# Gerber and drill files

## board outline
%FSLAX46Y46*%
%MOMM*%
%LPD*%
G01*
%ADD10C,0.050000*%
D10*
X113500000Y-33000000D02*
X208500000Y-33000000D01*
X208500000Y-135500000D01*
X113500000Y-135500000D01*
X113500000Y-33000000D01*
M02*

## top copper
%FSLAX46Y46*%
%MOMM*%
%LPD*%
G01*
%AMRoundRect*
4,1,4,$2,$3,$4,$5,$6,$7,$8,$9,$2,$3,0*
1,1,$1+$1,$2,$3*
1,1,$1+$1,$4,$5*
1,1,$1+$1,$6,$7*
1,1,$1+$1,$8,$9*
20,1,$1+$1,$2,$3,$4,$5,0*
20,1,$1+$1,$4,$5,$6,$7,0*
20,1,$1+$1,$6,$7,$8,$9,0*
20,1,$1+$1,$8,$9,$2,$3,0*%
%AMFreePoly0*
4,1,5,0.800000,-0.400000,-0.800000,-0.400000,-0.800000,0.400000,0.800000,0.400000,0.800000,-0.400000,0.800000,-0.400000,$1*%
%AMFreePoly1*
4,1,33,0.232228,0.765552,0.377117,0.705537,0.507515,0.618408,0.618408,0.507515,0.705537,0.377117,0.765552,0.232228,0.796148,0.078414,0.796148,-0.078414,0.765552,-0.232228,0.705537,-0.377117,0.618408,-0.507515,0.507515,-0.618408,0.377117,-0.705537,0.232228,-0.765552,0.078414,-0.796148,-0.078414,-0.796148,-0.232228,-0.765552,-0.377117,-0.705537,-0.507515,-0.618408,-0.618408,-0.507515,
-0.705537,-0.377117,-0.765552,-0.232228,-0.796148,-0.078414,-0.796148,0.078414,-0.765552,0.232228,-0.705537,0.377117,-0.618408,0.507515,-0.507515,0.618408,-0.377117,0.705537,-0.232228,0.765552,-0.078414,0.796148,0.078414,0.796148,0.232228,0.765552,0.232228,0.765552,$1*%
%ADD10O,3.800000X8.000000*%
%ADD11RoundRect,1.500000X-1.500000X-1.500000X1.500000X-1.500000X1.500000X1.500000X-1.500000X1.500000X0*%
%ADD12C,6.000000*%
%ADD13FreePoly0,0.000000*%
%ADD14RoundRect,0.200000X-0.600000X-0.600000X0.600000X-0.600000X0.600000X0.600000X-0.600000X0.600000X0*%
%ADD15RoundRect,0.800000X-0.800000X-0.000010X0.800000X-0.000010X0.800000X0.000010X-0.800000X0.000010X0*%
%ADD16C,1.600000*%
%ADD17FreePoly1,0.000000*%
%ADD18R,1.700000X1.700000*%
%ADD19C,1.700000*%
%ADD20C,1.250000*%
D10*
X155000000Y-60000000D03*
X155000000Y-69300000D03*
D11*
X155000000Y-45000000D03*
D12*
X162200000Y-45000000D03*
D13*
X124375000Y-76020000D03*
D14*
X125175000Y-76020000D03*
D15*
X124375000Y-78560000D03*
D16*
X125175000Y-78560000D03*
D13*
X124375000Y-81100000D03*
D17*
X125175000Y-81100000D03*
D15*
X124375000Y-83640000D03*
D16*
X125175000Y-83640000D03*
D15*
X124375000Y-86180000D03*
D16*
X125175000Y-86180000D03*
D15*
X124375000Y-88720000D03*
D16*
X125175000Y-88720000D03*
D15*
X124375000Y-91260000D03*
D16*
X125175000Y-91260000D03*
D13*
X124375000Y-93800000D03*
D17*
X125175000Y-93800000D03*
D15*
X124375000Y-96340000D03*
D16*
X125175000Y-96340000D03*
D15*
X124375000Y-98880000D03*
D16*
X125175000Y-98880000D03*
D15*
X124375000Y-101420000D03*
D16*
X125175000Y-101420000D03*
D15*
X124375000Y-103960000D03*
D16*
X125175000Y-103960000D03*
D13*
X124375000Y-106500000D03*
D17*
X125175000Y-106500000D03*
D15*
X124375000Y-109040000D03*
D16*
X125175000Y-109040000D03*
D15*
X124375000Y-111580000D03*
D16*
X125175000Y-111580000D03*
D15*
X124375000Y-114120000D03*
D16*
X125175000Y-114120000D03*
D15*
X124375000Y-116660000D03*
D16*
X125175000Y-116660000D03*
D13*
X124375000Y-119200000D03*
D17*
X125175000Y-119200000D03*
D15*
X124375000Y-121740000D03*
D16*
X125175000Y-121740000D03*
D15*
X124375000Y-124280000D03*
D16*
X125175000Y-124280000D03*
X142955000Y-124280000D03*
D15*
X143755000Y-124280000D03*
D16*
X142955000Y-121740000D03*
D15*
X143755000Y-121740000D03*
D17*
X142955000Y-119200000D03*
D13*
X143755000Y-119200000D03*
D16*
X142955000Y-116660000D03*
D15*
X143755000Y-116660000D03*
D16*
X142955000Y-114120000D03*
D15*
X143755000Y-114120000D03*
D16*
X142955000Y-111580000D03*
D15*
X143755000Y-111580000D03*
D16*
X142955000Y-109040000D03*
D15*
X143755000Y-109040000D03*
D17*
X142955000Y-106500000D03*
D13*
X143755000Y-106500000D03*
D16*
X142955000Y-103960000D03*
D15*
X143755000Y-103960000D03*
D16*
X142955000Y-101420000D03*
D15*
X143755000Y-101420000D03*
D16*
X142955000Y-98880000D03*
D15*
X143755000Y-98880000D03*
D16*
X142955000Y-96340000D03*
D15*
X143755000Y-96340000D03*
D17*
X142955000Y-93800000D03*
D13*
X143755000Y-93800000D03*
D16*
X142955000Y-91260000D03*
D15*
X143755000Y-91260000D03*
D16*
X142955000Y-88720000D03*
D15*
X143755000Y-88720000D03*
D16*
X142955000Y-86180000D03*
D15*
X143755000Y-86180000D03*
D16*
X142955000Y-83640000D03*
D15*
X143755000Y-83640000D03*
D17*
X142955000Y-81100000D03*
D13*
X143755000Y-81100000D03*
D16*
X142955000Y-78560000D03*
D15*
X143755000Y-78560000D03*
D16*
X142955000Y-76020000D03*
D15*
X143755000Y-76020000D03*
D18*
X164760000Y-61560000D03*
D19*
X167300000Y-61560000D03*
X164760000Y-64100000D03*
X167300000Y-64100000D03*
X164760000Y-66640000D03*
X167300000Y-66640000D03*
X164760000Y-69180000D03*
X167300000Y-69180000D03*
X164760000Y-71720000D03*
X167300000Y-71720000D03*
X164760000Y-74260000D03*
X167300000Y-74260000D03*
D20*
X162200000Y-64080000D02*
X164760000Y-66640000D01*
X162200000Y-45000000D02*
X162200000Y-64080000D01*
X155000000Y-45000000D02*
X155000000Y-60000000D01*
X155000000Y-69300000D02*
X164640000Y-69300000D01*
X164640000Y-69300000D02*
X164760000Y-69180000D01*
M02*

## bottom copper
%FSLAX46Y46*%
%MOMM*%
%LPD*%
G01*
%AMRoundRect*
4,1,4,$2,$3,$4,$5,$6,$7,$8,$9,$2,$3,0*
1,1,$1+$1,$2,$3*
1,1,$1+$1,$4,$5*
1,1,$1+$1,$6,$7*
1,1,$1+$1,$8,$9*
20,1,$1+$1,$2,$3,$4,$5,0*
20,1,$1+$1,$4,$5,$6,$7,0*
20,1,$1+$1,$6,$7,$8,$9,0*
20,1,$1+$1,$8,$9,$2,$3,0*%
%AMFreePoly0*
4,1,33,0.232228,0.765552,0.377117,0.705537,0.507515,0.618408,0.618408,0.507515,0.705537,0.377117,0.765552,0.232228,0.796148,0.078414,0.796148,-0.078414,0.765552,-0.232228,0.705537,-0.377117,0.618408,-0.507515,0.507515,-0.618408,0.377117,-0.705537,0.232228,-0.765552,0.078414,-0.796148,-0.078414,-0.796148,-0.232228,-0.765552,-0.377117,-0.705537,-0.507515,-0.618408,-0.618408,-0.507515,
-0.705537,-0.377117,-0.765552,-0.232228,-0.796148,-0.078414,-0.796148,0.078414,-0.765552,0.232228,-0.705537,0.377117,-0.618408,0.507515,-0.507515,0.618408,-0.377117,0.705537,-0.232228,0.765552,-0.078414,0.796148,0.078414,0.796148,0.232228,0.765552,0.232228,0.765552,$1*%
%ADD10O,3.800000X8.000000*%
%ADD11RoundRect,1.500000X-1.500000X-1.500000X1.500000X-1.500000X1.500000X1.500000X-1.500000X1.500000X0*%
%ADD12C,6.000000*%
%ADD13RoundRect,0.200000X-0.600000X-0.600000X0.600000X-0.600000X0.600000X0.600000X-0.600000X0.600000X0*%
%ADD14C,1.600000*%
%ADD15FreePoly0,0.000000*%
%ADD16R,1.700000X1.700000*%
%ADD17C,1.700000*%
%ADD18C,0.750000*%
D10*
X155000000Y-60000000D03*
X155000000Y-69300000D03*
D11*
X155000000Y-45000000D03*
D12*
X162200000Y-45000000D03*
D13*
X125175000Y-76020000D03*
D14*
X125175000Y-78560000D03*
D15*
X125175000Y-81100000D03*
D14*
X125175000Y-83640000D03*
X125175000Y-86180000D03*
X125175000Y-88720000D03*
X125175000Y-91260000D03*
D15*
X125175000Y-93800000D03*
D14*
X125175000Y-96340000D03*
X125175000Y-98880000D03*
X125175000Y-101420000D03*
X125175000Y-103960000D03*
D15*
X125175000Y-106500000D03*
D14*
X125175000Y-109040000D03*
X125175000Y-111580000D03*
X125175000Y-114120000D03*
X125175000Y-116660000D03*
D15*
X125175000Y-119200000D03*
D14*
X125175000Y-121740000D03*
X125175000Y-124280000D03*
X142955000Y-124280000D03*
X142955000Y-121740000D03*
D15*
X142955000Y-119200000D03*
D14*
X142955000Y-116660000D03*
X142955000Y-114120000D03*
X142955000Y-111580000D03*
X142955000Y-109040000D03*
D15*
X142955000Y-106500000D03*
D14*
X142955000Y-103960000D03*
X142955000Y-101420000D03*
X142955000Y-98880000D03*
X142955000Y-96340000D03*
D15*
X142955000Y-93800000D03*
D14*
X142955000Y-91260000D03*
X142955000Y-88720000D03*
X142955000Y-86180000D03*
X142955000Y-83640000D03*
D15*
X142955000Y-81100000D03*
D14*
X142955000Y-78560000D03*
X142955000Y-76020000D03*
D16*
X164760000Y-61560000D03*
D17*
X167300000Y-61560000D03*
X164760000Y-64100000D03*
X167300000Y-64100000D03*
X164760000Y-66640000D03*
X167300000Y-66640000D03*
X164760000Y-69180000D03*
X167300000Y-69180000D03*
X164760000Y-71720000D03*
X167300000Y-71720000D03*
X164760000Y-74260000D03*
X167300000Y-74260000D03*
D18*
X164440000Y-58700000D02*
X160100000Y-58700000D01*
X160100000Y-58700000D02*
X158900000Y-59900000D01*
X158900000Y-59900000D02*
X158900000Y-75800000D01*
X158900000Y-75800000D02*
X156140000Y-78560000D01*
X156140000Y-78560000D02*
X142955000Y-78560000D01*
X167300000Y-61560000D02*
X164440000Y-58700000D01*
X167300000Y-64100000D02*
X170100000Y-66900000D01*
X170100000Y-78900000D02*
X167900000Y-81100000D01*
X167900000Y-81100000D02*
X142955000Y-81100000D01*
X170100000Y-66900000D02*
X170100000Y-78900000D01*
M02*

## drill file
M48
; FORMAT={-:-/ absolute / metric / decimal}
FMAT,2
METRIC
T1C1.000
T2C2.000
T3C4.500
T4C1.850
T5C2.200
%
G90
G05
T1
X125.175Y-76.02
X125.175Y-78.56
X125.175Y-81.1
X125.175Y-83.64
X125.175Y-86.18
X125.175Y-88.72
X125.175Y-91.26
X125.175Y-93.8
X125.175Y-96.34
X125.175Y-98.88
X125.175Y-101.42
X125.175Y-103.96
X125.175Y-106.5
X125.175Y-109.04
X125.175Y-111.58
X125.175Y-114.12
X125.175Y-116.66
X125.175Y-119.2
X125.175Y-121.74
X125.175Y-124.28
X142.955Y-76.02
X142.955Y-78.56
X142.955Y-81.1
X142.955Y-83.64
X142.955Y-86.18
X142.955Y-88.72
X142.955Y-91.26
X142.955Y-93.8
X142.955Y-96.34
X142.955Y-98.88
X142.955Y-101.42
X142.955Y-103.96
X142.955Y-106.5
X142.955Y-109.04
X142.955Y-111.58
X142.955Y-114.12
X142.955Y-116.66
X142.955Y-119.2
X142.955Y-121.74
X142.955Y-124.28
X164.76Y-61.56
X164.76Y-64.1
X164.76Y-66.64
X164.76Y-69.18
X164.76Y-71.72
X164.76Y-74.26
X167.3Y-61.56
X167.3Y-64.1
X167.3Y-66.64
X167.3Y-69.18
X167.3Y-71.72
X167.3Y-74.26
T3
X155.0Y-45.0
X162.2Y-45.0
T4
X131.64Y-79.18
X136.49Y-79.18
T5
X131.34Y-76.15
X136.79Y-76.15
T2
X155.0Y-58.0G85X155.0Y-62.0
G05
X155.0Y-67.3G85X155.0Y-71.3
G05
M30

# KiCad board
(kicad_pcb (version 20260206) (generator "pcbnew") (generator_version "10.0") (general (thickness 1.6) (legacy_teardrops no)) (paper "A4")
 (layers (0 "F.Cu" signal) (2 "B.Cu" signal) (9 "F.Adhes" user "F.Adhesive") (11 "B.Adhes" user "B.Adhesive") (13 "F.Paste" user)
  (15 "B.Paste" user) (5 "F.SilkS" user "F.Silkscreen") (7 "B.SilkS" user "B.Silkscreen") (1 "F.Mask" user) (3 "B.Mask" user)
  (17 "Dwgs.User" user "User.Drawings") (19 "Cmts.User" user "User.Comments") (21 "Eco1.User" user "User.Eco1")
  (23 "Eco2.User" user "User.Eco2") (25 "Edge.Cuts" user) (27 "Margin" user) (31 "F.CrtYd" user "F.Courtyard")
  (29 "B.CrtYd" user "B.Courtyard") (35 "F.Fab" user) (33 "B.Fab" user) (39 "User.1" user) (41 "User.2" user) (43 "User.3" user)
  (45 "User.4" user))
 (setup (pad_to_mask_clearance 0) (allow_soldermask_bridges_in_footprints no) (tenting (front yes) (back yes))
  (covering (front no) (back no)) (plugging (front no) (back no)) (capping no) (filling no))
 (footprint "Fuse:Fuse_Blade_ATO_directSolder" (layer "F.Cu") (at 155 60 -90)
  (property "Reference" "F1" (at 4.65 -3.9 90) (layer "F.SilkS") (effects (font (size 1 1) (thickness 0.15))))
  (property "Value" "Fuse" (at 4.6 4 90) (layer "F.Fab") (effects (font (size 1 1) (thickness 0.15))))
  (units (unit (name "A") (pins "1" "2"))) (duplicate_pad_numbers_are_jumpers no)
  (pad "1" thru_hole oval (at 0 0 270) (size 8 3.8) (drill oval 6 2) (layers "*.Cu" "*.Mask") (remove_unused_layers no) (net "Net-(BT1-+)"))
  (pad "2" thru_hole oval (at 9.3 0 270) (size 8 3.8) (drill oval 6 2) (layers "*.Cu" "*.Mask") (remove_unused_layers no)
   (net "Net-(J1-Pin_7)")))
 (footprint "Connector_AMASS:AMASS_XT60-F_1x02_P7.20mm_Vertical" (layer "F.Cu") (at 155 45)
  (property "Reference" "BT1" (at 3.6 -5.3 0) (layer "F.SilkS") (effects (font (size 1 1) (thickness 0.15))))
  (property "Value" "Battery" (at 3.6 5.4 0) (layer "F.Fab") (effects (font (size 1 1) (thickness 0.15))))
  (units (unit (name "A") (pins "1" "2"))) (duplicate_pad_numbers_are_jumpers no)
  (pad "1" thru_hole roundrect (at 0 0) (size 6 6) (drill 4.5) (layers "*.Cu" "*.Mask") (remove_unused_layers no) (roundrect_rratio 0.25)
   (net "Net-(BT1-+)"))
  (pad "2" thru_hole circle (at 7.2 0) (size 6 6) (drill 4.5) (layers "*.Cu" "*.Mask") (remove_unused_layers no) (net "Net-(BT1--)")))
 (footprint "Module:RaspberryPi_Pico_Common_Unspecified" (layer "F.Cu") (at 134.065 100.15)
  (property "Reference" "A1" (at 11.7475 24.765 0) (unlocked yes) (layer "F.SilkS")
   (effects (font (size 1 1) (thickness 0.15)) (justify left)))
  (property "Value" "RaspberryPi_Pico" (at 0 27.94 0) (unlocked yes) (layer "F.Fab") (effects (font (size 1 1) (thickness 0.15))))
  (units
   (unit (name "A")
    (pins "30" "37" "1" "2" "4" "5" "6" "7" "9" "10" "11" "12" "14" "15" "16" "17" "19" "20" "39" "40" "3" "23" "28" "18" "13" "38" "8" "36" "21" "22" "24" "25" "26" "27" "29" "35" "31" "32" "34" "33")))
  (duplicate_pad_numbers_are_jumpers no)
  (pad "" np_thru_hole circle (at -2.725 -24) (size 2.2 2.2) (drill 2.2) (layers "*.Mask"))
  (pad "" np_thru_hole circle (at -2.425 -20.97) (size 1.85 1.85) (drill 1.85) (layers "*.Mask"))
  (pad "" np_thru_hole circle (at 2.425 -20.97) (size 1.85 1.85) (drill 1.85) (layers "*.Mask"))
  (pad "" np_thru_hole circle (at 2.725 -24) (size 2.2 2.2) (drill 2.2) (layers "*.Mask"))
  (pad "1" smd custom (at -9.69 -24.13) (size 1.6 0.8) (layers "F.Cu" "F.Mask") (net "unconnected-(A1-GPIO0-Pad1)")
   (options (clearance outline) (anchor rect)) (primitives))
  (pad "1" thru_hole roundrect (at -8.89 -24.13) (size 1.6 1.6) (drill 1) (layers "*.Cu" "*.Mask") (remove_unused_layers no)
   (roundrect_rratio 0.125) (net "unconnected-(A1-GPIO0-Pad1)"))
  (pad "2" smd roundrect (at -9.69 -21.59) (size 3.2 1.6) (layers "F.Cu" "F.Mask") (roundrect_rratio 0.5)
   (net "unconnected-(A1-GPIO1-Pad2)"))
  (pad "2" thru_hole circle (at -8.89 -21.59) (size 1.6 1.6) (drill 1) (layers "*.Cu" "*.Mask") (remove_unused_layers no)
   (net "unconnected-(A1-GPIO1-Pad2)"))
  (pad "3" smd custom (at -9.69 -19.05) (size 1.6 0.8) (layers "F.Cu" "F.Mask") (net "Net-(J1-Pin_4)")
   (options (clearance outline) (anchor rect)) (primitives))
  (pad "3" thru_hole custom (at -8.89 -19.05) (size 1.6 1.6) (drill 1) (layers "*.Cu" "*.Mask") (remove_unused_layers no)
   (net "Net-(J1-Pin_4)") (options (clearance outline) (anchor circle)) (primitives))
  (pad "4" smd roundrect (at -9.69 -16.51) (size 3.2 1.6) (layers "F.Cu" "F.Mask") (roundrect_rratio 0.5)
   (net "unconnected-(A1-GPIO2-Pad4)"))
  (pad "4" thru_hole circle (at -8.89 -16.51) (size 1.6 1.6) (drill 1) (layers "*.Cu" "*.Mask") (remove_unused_layers no)
   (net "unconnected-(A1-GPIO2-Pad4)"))
  (pad "5" smd roundrect (at -9.69 -13.97) (size 3.2 1.6) (layers "F.Cu" "F.Mask") (roundrect_rratio 0.5)
   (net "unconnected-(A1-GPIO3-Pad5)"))
  (pad "5" thru_hole circle (at -8.89 -13.97) (size 1.6 1.6) (drill 1) (layers "*.Cu" "*.Mask") (remove_unused_layers no)
   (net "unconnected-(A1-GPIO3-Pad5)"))
  (pad "6" smd roundrect (at -9.69 -11.43) (size 3.2 1.6) (layers "F.Cu" "F.Mask") (roundrect_rratio 0.5)
   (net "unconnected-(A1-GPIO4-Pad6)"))
  (pad "6" thru_hole circle (at -8.89 -11.43) (size 1.6 1.6) (drill 1) (layers "*.Cu" "*.Mask") (remove_unused_layers no)
   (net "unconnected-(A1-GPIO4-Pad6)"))
  (pad "7" smd roundrect (at -9.69 -8.89) (size 3.2 1.6) (layers "F.Cu" "F.Mask") (roundrect_rratio 0.5) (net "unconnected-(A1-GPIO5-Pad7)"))
  (pad "7" thru_hole circle (at -8.89 -8.89) (size 1.6 1.6) (drill 1) (layers "*.Cu" "*.Mask") (remove_unused_layers no)
   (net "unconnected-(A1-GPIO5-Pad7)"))
  (pad "8" smd custom (at -9.69 -6.35) (size 1.6 0.8) (layers "F.Cu" "F.Mask") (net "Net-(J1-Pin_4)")
   (options (clearance outline) (anchor rect)) (primitives))
  (pad "8" thru_hole custom (at -8.89 -6.35) (size 1.6 1.6) (drill 1) (layers "*.Cu" "*.Mask") (remove_unused_layers no)
   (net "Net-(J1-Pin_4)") (options (clearance outline) (anchor circle)) (primitives))
  (pad "9" smd roundrect (at -9.69 -3.81) (size 3.2 1.6) (layers "F.Cu" "F.Mask") (roundrect_rratio 0.5) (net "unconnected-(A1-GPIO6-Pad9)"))
  (pad "9" thru_hole circle (at -8.89 -3.81) (size 1.6 1.6) (drill 1) (layers "*.Cu" "*.Mask") (remove_unused_layers no)
   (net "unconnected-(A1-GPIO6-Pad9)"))
  (pad "10" smd roundrect (at -9.69 -1.27) (size 3.2 1.6) (layers "F.Cu" "F.Mask") (roundrect_rratio 0.5)
   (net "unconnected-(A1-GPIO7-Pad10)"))
  (pad "10" thru_hole circle (at -8.89 -1.27) (size 1.6 1.6) (drill 1) (layers "*.Cu" "*.Mask") (remove_unused_layers no)
   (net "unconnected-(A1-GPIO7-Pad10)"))
  (pad "11" smd roundrect (at -9.69 1.27) (size 3.2 1.6) (layers "F.Cu" "F.Mask") (roundrect_rratio 0.5)
   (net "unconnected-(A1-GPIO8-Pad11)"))
  (pad "11" thru_hole circle (at -8.89 1.27) (size 1.6 1.6) (drill 1) (layers "*.Cu" "*.Mask") (remove_unused_layers no)
   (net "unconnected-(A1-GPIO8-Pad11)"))
  (pad "12" smd roundrect (at -9.69 3.81) (size 3.2 1.6) (layers "F.Cu" "F.Mask") (roundrect_rratio 0.5)
   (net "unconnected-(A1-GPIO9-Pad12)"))
  (pad "12" thru_hole circle (at -8.89 3.81) (size 1.6 1.6) (drill 1) (layers "*.Cu" "*.Mask") (remove_unused_layers no)
   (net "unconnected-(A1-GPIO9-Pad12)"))
  (pad "13" smd custom (at -9.69 6.35) (size 1.6 0.8) (layers "F.Cu" "F.Mask") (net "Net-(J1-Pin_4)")
   (options (clearance outline) (anchor rect)) (primitives))
  (pad "13" thru_hole custom (at -8.89 6.35) (size 1.6 1.6) (drill 1) (layers "*.Cu" "*.Mask") (remove_unused_layers no)
   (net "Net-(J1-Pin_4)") (options (clearance outline) (anchor circle)) (primitives))
  (pad "14" smd roundrect (at -9.69 8.89) (size 3.2 1.6) (layers "F.Cu" "F.Mask") (roundrect_rratio 0.5)
   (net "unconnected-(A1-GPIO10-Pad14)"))
  (pad "14" thru_hole circle (at -8.89 8.89) (size 1.6 1.6) (drill 1) (layers "*.Cu" "*.Mask") (remove_unused_layers no)
   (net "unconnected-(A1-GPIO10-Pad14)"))
  (pad "15" smd roundrect (at -9.69 11.43) (size 3.2 1.6) (layers "F.Cu" "F.Mask") (roundrect_rratio 0.5)
   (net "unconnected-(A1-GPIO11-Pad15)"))
  (pad "15" thru_hole circle (at -8.89 11.43) (size 1.6 1.6) (drill 1) (layers "*.Cu" "*.Mask") (remove_unused_layers no)
   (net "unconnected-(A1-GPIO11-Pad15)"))
  (pad "16" smd roundrect (at -9.69 13.97) (size 3.2 1.6) (layers "F.Cu" "F.Mask") (roundrect_rratio 0.5)
   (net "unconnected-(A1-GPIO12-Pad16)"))
  (pad "16" thru_hole circle (at -8.89 13.97) (size 1.6 1.6) (drill 1) (layers "*.Cu" "*.Mask") (remove_unused_layers no)
   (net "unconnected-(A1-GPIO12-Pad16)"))
  (pad "17" smd roundrect (at -9.69 16.51) (size 3.2 1.6) (layers "F.Cu" "F.Mask") (roundrect_rratio 0.5)
   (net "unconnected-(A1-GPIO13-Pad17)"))
  (pad "17" thru_hole circle (at -8.89 16.51) (size 1.6 1.6) (drill 1) (layers "*.Cu" "*.Mask") (remove_unused_layers no)
   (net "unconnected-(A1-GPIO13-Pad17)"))
  (pad "18" smd custom (at -9.69 19.05) (size 1.6 0.8) (layers "F.Cu" "F.Mask") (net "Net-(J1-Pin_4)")
   (options (clearance outline) (anchor rect)) (primitives))
  (pad "18" thru_hole custom (at -8.89 19.05) (size 1.6 1.6) (drill 1) (layers "*.Cu" "*.Mask") (remove_unused_layers no)
   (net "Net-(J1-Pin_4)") (options (clearance outline) (anchor circle)) (primitives))
  (pad "19" smd roundrect (at -9.69 21.59) (size 3.2 1.6) (layers "F.Cu" "F.Mask") (roundrect_rratio 0.5)
   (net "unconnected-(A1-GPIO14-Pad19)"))
  (pad "19" thru_hole circle (at -8.89 21.59) (size 1.6 1.6) (drill 1) (layers "*.Cu" "*.Mask") (remove_unused_layers no)
   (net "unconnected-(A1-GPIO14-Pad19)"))
  (pad "20" smd roundrect (at -9.69 24.13) (size 3.2 1.6) (layers "F.Cu" "F.Mask") (roundrect_rratio 0.5)
   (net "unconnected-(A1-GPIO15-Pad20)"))
  (pad "20" thru_hole circle (at -8.89 24.13) (size 1.6 1.6) (drill 1) (layers "*.Cu" "*.Mask") (remove_unused_layers no)
   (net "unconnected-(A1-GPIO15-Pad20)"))
  (pad "21" thru_hole circle (at 8.89 24.13) (size 1.6 1.6) (drill 1) (layers "*.Cu" "*.Mask") (remove_unused_layers no)
   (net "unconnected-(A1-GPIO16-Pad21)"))
  (pad "21" smd roundrect (at 9.69 24.13) (size 3.2 1.6) (layers "F.Cu" "F.Mask") (roundrect_rratio 0.5)
   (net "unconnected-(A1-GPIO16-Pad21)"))
  (pad "22" thru_hole circle (at 8.89 21.59) (size 1.6 1.6) (drill 1) (layers "*.Cu" "*.Mask") (remove_unused_layers no)
   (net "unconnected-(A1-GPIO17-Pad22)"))
  (pad "22" smd roundrect (at 9.69 21.59) (size 3.2 1.6) (layers "F.Cu" "F.Mask") (roundrect_rratio 0.5)
   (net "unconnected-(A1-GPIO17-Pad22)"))
  (pad "23" thru_hole custom (at 8.89 19.05) (size 1.6 1.6) (drill 1) (layers "*.Cu" "*.Mask") (remove_unused_layers no)
   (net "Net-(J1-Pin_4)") (options (clearance outline) (anchor circle)) (primitives))
  (pad "23" smd custom (at 9.69 19.05) (size 1.6 0.8) (layers "F.Cu" "F.Mask") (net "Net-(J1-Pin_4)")
   (options (clearance outline) (anchor rect)) (primitives))
  (pad "24" thru_hole circle (at 8.89 16.51) (size 1.6 1.6) (drill 1) (layers "*.Cu" "*.Mask") (remove_unused_layers no)
   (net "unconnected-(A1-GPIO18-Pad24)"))
  (pad "24" smd roundrect (at 9.69 16.51) (size 3.2 1.6) (layers "F.Cu" "F.Mask") (roundrect_rratio 0.5)
   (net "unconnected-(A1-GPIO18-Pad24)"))
  (pad "25" thru_hole circle (at 8.89 13.97) (size 1.6 1.6) (drill 1) (layers "*.Cu" "*.Mask") (remove_unused_layers no)
   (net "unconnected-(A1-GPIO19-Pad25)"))
  (pad "25" smd roundrect (at 9.69 13.97) (size 3.2 1.6) (layers "F.Cu" "F.Mask") (roundrect_rratio 0.5)
   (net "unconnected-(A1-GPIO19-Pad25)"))
  (pad "26" thru_hole circle (at 8.89 11.43) (size 1.6 1.6) (drill 1) (layers "*.Cu" "*.Mask") (remove_unused_layers no)
   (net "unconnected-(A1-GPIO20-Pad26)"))
  (pad "26" smd roundrect (at 9.69 11.43) (size 3.2 1.6) (layers "F.Cu" "F.Mask") (roundrect_rratio 0.5)
   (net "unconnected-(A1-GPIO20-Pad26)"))
  (pad "27" thru_hole circle (at 8.89 8.89) (size 1.6 1.6) (drill 1) (layers "*.Cu" "*.Mask") (remove_unused_layers no)
   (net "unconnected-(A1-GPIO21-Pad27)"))
  (pad "27" smd roundrect (at 9.69 8.89) (size 3.2 1.6) (layers "F.Cu" "F.Mask") (roundrect_rratio 0.5)
   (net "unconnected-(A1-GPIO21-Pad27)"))
  (pad "28" thru_hole custom (at 8.89 6.35) (size 1.6 1.6) (drill 1) (layers "*.Cu" "*.Mask") (remove_unused_layers no)
   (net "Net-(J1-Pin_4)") (options (clearance outline) (anchor circle)) (primitives))
  (pad "28" smd custom (at 9.69 6.35) (size 1.6 0.8) (layers "F.Cu" "F.Mask") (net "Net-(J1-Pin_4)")
   (options (clearance outline) (anchor rect)) (primitives))
  (pad "29" thru_hole circle (at 8.89 3.81) (size 1.6 1.6) (drill 1) (layers "*.Cu" "*.Mask") (remove_unused_layers no)
   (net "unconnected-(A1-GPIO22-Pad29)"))
  (pad "29" smd roundrect (at 9.69 3.81) (size 3.2 1.6) (layers "F.Cu" "F.Mask") (roundrect_rratio 0.5)
   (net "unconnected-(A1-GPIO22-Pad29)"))
  (pad "30" thru_hole circle (at 8.89 1.27) (size 1.6 1.6) (drill 1) (layers "*.Cu" "*.Mask") (remove_unused_layers no)
   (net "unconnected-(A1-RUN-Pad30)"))
  (pad "30" smd roundrect (at 9.69 1.27) (size 3.2 1.6) (layers "F.Cu" "F.Mask") (roundrect_rratio 0.5) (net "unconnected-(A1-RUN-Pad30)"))
  (pad "31" thru_hole circle (at 8.89 -1.27) (size 1.6 1.6) (drill 1) (layers "*.Cu" "*.Mask") (remove_unused_layers no)
   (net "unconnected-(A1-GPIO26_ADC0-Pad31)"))
  (pad "31" smd roundrect (at 9.69 -1.27) (size 3.2 1.6) (layers "F.Cu" "F.Mask") (roundrect_rratio 0.5)
   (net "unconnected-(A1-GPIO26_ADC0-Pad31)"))
  (pad "32" thru_hole circle (at 8.89 -3.81) (size 1.6 1.6) (drill 1) (layers "*.Cu" "*.Mask") (remove_unused_layers no)
   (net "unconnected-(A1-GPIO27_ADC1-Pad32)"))
  (pad "32" smd roundrect (at 9.69 -3.81) (size 3.2 1.6) (layers "F.Cu" "F.Mask") (roundrect_rratio 0.5)
   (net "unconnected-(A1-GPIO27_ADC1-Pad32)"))
  (pad "33" thru_hole custom (at 8.89 -6.35) (size 1.6 1.6) (drill 1) (layers "*.Cu" "*.Mask") (remove_unused_layers no)
   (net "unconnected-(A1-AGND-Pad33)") (options (clearance outline) (anchor circle)) (primitives))
  (pad "33" smd custom (at 9.69 -6.35) (size 1.6 0.8) (layers "F.Cu" "F.Mask") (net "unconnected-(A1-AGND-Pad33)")
   (options (clearance outline) (anchor rect)) (primitives))
  (pad "34" thru_hole circle (at 8.89 -8.89) (size 1.6 1.6) (drill 1) (layers "*.Cu" "*.Mask") (remove_unused_layers no)
   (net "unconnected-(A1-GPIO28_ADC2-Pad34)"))
  (pad "34" smd roundrect (at 9.69 -8.89) (size 3.2 1.6) (layers "F.Cu" "F.Mask") (roundrect_rratio 0.5)
   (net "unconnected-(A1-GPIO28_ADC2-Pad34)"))
  (pad "35" thru_hole circle (at 8.89 -11.43) (size 1.6 1.6) (drill 1) (layers "*.Cu" "*.Mask") (remove_unused_layers no)
   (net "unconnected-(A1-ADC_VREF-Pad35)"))
  (pad "35" smd roundrect (at 9.69 -11.43) (size 3.2 1.6) (layers "F.Cu" "F.Mask") (roundrect_rratio 0.5)
   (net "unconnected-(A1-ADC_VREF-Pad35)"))
  (pad "36" thru_hole circle (at 8.89 -13.97) (size 1.6 1.6) (drill 1) (layers "*.Cu" "*.Mask") (remove_unused_layers no)
   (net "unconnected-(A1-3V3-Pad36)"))
  (pad "36" smd roundrect (at 9.69 -13.97) (size 3.2 1.6) (layers "F.Cu" "F.Mask") (roundrect_rratio 0.5) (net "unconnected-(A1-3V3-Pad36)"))
  (pad "37" thru_hole circle (at 8.89 -16.51) (size 1.6 1.6) (drill 1) (layers "*.Cu" "*.Mask") (remove_unused_layers no)
   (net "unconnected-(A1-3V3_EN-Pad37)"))
  (pad "37" smd roundrect (at 9.69 -16.51) (size 3.2 1.6) (layers "F.Cu" "F.Mask") (roundrect_rratio 0.5)
   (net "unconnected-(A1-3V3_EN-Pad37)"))
  (pad "38" thru_hole custom (at 8.89 -19.05) (size 1.6 1.6) (drill 1) (layers "*.Cu" "*.Mask") (remove_unused_layers no)
   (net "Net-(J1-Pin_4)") (options (clearance outline) (anchor circle)) (primitives))
  (pad "38" smd custom (at 9.69 -19.05) (size 1.6 0.8) (layers "F.Cu" "F.Mask") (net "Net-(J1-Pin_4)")
   (options (clearance outline) (anchor rect)) (primitives))
  (pad "39" thru_hole circle (at 8.89 -21.59) (size 1.6 1.6) (drill 1) (layers "*.Cu" "*.Mask") (remove_unused_layers no)
   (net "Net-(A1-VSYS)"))
  (pad "39" smd roundrect (at 9.69 -21.59) (size 3.2 1.6) (layers "F.Cu" "F.Mask") (roundrect_rratio 0.5) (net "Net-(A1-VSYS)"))
  (pad "40" thru_hole circle (at 8.89 -24.13) (size 1.6 1.6) (drill 1) (layers "*.Cu" "*.Mask") (remove_unused_layers no)
   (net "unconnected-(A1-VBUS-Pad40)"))
  (pad "40" smd roundrect (at 9.69 -24.13) (size 3.2 1.6) (layers "F.Cu" "F.Mask") (roundrect_rratio 0.5)
   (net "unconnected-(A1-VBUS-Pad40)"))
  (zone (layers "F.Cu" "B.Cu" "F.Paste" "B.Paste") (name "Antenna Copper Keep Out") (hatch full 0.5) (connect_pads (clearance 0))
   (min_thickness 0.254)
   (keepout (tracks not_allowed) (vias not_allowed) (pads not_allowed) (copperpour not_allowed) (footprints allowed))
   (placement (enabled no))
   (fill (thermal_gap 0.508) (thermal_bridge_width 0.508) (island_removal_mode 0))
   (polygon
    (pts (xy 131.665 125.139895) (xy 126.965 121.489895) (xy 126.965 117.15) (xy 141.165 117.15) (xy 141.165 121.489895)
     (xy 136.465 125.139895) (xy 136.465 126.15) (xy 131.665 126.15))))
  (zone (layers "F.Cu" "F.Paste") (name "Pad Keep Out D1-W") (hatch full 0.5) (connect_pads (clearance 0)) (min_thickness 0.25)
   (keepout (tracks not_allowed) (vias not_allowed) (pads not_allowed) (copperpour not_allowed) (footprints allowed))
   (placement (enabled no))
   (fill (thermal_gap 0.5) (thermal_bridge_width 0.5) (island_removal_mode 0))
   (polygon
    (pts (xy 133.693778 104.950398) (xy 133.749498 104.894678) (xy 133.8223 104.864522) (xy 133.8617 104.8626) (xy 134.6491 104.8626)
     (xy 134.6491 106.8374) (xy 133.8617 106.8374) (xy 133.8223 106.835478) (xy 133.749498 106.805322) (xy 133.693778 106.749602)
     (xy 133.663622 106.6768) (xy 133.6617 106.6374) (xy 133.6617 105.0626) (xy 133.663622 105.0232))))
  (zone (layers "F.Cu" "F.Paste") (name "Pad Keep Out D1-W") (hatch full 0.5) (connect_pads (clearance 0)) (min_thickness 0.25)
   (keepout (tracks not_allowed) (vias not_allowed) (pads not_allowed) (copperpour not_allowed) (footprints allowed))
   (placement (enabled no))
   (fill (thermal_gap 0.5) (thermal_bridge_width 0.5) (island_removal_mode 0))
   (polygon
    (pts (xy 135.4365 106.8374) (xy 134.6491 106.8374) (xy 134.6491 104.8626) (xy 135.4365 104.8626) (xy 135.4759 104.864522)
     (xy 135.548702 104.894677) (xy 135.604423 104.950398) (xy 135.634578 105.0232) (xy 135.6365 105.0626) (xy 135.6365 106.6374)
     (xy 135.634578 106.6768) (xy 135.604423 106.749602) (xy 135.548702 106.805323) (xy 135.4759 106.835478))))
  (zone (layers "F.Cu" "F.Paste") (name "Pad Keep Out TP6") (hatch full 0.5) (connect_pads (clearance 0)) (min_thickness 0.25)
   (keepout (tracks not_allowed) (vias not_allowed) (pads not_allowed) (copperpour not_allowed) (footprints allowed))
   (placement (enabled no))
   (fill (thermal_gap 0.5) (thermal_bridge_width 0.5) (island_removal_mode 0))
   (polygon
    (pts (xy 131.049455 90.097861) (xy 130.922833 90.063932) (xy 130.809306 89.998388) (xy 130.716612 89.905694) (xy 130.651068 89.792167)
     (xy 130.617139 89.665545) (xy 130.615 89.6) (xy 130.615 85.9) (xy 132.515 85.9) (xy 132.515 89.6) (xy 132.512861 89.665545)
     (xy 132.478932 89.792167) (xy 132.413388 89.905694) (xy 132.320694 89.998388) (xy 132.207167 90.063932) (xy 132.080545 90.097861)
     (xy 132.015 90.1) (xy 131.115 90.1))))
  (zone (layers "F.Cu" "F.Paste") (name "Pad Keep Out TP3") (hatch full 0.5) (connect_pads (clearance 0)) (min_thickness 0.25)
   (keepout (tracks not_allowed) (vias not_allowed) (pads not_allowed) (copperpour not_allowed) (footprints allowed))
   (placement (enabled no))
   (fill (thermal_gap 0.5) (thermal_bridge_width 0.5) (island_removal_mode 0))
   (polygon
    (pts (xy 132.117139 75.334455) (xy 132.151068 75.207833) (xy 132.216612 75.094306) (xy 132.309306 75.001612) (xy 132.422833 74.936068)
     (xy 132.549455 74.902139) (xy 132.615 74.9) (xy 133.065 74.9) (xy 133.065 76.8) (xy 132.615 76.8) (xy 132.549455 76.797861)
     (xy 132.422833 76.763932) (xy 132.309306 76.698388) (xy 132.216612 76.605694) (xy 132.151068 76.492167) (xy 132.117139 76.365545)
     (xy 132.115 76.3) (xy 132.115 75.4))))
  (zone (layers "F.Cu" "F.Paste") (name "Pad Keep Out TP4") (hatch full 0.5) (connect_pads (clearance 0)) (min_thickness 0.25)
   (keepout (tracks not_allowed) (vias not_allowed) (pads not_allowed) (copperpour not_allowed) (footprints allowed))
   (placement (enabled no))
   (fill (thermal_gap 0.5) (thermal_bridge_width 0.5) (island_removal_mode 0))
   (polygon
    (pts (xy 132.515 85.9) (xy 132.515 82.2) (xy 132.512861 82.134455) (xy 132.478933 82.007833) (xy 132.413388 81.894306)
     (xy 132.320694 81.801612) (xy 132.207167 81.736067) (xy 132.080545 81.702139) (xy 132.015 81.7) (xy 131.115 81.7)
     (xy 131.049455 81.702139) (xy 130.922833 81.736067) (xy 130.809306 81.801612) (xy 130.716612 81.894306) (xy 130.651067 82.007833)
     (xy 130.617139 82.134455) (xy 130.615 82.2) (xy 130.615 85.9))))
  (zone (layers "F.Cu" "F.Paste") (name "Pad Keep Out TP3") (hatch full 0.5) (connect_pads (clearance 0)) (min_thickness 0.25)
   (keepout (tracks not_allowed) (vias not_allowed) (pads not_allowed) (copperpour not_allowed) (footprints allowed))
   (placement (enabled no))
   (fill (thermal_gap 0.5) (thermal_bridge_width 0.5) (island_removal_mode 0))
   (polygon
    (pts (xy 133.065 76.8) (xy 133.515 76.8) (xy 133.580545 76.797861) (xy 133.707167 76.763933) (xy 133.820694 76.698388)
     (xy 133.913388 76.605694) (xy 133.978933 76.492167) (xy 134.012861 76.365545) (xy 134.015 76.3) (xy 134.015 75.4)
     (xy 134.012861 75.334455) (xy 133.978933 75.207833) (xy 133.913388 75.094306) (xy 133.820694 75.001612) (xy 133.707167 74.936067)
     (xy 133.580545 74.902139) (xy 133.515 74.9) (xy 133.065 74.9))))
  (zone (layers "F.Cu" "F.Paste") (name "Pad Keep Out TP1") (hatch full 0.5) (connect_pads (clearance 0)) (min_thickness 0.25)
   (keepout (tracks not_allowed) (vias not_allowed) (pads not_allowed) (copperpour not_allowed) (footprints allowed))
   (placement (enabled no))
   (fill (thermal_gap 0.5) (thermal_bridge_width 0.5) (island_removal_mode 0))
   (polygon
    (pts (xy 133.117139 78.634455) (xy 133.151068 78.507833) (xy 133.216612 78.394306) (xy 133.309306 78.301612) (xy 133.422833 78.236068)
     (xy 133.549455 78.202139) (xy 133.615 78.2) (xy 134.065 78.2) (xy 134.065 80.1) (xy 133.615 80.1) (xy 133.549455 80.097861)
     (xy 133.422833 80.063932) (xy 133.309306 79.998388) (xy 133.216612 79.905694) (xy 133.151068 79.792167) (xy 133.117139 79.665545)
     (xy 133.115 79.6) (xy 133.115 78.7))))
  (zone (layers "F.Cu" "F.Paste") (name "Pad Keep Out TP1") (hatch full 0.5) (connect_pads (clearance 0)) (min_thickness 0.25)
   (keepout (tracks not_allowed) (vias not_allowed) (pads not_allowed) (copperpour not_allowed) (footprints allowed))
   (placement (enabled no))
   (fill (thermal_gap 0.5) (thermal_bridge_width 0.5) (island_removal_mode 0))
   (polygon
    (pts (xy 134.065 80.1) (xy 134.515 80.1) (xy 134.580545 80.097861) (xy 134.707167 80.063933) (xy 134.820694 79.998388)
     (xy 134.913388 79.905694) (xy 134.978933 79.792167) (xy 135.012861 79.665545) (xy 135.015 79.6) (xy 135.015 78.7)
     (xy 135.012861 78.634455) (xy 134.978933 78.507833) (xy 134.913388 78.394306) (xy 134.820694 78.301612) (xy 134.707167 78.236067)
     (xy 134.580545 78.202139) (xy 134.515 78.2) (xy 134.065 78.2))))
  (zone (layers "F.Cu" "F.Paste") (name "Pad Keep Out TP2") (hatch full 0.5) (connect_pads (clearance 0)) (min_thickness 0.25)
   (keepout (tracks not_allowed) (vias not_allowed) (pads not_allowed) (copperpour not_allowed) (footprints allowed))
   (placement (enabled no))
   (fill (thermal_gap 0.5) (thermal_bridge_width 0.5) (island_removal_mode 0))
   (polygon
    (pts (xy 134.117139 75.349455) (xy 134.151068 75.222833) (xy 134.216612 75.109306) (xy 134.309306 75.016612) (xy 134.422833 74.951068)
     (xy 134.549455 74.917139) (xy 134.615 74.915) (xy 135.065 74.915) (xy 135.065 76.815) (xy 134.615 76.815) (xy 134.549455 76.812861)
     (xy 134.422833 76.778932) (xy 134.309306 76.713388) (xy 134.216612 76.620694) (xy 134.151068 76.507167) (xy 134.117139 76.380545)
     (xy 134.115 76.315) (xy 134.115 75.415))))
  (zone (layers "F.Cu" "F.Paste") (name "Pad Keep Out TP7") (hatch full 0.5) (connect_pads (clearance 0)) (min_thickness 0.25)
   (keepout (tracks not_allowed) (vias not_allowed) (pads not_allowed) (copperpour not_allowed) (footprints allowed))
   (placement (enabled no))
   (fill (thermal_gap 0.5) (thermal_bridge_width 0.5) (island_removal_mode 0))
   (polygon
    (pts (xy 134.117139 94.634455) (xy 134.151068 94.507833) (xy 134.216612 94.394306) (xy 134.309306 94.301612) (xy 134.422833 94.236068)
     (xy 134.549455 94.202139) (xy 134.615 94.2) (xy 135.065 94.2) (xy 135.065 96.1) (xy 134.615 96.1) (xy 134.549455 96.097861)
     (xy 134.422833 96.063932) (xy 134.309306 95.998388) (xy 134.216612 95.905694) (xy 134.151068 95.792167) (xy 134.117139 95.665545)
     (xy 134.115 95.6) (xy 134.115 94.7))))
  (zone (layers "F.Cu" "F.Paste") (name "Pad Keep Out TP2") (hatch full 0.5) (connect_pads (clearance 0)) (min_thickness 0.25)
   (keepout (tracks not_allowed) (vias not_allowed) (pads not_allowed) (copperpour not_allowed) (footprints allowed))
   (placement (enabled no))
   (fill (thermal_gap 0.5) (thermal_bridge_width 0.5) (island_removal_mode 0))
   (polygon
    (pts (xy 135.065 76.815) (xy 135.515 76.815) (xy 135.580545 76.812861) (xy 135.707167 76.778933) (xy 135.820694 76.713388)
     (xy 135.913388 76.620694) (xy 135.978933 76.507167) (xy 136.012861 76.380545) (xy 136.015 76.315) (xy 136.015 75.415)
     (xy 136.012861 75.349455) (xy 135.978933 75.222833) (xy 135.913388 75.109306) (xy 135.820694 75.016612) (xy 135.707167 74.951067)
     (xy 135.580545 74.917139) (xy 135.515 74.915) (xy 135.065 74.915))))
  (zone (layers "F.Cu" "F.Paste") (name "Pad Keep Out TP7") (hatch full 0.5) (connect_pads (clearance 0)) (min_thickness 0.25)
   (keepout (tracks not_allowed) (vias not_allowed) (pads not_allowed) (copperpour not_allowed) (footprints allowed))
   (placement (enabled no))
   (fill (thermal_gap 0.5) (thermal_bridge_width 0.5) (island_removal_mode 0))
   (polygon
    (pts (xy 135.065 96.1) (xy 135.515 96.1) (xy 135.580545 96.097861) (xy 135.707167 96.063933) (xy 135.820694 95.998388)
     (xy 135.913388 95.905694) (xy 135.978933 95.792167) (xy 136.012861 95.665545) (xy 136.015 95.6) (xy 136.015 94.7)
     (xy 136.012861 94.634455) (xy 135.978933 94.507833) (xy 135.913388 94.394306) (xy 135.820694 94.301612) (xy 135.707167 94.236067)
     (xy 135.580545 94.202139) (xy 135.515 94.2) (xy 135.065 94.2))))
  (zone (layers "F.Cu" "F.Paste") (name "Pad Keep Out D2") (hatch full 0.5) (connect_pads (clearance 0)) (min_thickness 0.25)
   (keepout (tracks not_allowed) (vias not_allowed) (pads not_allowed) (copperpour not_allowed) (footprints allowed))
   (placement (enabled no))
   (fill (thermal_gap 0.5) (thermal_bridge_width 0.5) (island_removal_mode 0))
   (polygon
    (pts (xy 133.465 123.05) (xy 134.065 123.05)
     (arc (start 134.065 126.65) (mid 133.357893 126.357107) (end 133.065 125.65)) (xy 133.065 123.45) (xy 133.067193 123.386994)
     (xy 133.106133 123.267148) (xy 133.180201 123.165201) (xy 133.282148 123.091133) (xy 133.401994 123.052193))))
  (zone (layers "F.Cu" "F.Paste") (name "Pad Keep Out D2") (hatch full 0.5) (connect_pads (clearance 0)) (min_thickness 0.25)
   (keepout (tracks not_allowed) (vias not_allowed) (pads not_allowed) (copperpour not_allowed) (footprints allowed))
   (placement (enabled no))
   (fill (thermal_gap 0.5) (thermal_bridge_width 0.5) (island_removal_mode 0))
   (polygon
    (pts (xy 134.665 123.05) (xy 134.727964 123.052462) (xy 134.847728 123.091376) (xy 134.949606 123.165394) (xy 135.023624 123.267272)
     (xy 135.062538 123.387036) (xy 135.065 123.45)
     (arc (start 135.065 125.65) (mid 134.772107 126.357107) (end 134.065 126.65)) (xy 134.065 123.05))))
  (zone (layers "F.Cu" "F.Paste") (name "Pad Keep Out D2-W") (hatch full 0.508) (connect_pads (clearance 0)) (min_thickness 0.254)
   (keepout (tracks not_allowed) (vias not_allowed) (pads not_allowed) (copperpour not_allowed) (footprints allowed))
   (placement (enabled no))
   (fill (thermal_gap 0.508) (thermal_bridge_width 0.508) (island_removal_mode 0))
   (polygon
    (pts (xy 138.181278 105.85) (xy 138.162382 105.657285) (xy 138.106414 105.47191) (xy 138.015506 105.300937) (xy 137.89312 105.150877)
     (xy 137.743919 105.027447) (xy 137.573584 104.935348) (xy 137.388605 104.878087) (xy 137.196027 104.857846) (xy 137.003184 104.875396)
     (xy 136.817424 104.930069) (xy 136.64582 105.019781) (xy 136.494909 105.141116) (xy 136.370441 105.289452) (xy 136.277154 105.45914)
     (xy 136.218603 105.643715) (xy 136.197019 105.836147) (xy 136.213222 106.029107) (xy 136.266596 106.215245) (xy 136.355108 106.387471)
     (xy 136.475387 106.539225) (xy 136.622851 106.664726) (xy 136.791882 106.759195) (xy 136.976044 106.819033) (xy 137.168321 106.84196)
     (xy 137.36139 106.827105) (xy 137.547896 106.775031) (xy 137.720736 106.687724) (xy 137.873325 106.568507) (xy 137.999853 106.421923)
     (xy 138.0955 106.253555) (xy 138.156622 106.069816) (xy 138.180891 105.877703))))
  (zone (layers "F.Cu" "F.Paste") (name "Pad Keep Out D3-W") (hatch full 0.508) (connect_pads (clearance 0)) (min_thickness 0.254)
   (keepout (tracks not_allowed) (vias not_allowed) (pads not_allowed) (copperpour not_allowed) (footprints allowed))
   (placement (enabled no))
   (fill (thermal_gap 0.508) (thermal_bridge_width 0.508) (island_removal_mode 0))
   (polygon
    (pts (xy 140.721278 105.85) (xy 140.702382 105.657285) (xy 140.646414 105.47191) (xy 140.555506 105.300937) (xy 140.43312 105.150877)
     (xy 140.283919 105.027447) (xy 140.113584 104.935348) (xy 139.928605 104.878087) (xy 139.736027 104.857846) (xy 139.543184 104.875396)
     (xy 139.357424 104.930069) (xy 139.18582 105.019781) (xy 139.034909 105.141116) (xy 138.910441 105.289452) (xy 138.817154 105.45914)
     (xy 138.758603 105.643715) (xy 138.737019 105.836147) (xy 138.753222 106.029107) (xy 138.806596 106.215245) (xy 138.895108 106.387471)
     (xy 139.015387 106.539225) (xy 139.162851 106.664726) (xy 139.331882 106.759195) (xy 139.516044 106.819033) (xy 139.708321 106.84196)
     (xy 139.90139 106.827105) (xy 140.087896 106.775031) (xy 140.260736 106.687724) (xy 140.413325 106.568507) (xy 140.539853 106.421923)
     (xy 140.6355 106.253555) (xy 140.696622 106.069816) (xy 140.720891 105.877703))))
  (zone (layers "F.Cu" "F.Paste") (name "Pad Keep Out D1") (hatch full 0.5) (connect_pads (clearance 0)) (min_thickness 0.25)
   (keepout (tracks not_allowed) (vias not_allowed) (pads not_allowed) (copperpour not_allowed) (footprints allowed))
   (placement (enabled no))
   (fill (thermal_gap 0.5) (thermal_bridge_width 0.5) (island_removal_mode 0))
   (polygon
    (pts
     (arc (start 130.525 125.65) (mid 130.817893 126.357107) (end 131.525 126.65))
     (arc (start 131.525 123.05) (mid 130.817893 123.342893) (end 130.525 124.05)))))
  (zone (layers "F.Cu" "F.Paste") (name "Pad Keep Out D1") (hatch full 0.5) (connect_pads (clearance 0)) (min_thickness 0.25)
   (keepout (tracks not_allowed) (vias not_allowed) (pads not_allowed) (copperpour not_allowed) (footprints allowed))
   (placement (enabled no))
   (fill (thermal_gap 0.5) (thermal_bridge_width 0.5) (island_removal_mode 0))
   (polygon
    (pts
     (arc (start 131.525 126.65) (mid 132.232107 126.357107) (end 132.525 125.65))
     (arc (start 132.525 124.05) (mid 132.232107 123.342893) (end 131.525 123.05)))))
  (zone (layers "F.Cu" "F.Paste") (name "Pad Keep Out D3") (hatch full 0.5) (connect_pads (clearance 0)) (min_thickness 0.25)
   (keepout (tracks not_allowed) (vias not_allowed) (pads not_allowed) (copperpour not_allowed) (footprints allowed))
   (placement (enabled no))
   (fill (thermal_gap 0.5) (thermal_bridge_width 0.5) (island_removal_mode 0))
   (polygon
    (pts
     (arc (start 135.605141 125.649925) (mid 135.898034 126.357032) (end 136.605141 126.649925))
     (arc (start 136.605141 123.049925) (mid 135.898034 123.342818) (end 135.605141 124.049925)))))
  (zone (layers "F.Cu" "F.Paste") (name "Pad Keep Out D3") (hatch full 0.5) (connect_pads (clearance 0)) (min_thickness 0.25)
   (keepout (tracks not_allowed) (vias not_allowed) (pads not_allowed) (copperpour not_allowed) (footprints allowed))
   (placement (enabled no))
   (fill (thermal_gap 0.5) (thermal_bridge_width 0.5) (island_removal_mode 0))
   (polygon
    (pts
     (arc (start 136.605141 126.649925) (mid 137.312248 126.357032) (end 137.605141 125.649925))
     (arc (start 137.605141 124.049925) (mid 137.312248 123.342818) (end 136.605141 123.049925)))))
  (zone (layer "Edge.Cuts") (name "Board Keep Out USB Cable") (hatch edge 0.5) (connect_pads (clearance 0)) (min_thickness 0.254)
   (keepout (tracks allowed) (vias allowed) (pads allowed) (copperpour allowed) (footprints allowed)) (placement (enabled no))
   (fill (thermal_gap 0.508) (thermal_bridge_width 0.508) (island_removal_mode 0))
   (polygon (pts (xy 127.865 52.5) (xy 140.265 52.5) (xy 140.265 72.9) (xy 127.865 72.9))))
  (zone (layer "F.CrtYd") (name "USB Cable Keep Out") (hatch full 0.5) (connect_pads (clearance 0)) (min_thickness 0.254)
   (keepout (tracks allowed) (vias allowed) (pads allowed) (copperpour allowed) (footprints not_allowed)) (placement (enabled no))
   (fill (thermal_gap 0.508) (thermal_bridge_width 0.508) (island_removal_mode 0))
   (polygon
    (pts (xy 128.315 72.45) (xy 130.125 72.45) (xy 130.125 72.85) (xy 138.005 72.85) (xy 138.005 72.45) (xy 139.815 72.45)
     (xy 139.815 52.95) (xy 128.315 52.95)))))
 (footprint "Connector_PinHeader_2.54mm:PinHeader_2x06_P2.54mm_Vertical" (layer "F.Cu") (at 164.76 61.56)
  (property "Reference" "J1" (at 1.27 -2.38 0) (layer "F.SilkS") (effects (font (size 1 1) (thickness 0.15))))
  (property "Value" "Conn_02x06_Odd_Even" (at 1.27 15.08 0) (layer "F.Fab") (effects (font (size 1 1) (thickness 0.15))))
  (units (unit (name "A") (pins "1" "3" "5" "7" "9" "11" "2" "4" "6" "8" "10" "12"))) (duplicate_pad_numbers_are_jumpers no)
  (pad "1" thru_hole rect (at 0 0) (size 1.7 1.7) (drill 1) (layers "*.Cu" "*.Mask") (remove_unused_layers no)
   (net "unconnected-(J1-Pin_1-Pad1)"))
  (pad "2" thru_hole circle (at 2.54 0) (size 1.7 1.7) (drill 1) (layers "*.Cu" "*.Mask") (remove_unused_layers no) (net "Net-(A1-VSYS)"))
  (pad "3" thru_hole circle (at 0 2.54) (size 1.7 1.7) (drill 1) (layers "*.Cu" "*.Mask") (remove_unused_layers no)
   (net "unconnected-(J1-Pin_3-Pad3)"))
  (pad "4" thru_hole circle (at 2.54 2.54) (size 1.7 1.7) (drill 1) (layers "*.Cu" "*.Mask") (remove_unused_layers no)
   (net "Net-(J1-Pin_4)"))
  (pad "5" thru_hole circle (at 0 5.08) (size 1.7 1.7) (drill 1) (layers "*.Cu" "*.Mask") (remove_unused_layers no) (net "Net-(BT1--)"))
  (pad "6" thru_hole circle (at 2.54 5.08) (size 1.7 1.7) (drill 1) (layers "*.Cu" "*.Mask") (remove_unused_layers no)
   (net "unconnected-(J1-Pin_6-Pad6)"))
  (pad "7" thru_hole circle (at 0 7.62) (size 1.7 1.7) (drill 1) (layers "*.Cu" "*.Mask") (remove_unused_layers no) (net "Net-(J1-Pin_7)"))
  (pad "8" thru_hole circle (at 2.54 7.62) (size 1.7 1.7) (drill 1) (layers "*.Cu" "*.Mask") (remove_unused_layers no)
   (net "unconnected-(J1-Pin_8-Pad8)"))
  (pad "9" thru_hole circle (at 0 10.16) (size 1.7 1.7) (drill 1) (layers "*.Cu" "*.Mask") (remove_unused_layers no)
   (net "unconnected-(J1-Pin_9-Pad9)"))
  (pad "10" thru_hole circle (at 2.54 10.16) (size 1.7 1.7) (drill 1) (layers "*.Cu" "*.Mask") (remove_unused_layers no)
   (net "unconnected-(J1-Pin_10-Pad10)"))
  (pad "11" thru_hole circle (at 0 12.7) (size 1.7 1.7) (drill 1) (layers "*.Cu" "*.Mask") (remove_unused_layers no)
   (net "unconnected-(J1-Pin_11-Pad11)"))
  (pad "12" thru_hole circle (at 2.54 12.7) (size 1.7 1.7) (drill 1) (layers "*.Cu" "*.Mask") (remove_unused_layers no)
   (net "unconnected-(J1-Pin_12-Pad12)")))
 (gr_rect (start 113.5 33) (end 208.5 135.5) (stroke (width 0.05) (type default)) (fill no) (layer "Edge.Cuts"))
 (segment (start 164.44 58.7) (end 160.1 58.7) (width 0.75) (layer "B.Cu") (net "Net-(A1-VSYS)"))
 (segment (start 160.1 58.7) (end 158.9 59.9) (width 0.75) (layer "B.Cu") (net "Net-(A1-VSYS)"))
 (segment (start 158.9 59.9) (end 158.9 75.8) (width 0.75) (layer "B.Cu") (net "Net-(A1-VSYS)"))
 (segment (start 158.9 75.8) (end 156.14 78.56) (width 0.75) (layer "B.Cu") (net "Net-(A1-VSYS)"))
 (segment (start 156.14 78.56) (end 142.955 78.56) (width 0.75) (layer "B.Cu") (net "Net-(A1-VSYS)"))
 (segment (start 167.3 61.56) (end 164.44 58.7) (width 0.75) (layer "B.Cu") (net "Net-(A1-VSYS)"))
 (segment (start 162.2 64.08) (end 164.76 66.64) (width 1.25) (layer "F.Cu") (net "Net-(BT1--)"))
 (segment (start 162.2 45) (end 162.2 64.08) (width 1.25) (layer "F.Cu") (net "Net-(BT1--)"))
 (segment (start 155 45) (end 155 60) (width 1.25) (layer "F.Cu") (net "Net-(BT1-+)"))
 (segment (start 167.3 64.1) (end 170.1 66.9) (width 0.75) (layer "B.Cu") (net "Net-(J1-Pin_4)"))
 (segment (start 170.1 78.9) (end 167.9 81.1) (width 0.75) (layer "B.Cu") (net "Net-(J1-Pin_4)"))
 (segment (start 167.9 81.1) (end 142.955 81.1) (width 0.75) (layer "B.Cu") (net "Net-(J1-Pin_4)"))
 (segment (start 170.1 66.9) (end 170.1 78.9) (width 0.75) (layer "B.Cu") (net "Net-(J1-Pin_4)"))
 (segment (start 155 69.3) (end 164.64 69.3) (width 1.25) (layer "F.Cu") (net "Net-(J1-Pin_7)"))
 (segment (start 164.64 69.3) (end 164.76 69.18) (width 1.25) (layer "F.Cu") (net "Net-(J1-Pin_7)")))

